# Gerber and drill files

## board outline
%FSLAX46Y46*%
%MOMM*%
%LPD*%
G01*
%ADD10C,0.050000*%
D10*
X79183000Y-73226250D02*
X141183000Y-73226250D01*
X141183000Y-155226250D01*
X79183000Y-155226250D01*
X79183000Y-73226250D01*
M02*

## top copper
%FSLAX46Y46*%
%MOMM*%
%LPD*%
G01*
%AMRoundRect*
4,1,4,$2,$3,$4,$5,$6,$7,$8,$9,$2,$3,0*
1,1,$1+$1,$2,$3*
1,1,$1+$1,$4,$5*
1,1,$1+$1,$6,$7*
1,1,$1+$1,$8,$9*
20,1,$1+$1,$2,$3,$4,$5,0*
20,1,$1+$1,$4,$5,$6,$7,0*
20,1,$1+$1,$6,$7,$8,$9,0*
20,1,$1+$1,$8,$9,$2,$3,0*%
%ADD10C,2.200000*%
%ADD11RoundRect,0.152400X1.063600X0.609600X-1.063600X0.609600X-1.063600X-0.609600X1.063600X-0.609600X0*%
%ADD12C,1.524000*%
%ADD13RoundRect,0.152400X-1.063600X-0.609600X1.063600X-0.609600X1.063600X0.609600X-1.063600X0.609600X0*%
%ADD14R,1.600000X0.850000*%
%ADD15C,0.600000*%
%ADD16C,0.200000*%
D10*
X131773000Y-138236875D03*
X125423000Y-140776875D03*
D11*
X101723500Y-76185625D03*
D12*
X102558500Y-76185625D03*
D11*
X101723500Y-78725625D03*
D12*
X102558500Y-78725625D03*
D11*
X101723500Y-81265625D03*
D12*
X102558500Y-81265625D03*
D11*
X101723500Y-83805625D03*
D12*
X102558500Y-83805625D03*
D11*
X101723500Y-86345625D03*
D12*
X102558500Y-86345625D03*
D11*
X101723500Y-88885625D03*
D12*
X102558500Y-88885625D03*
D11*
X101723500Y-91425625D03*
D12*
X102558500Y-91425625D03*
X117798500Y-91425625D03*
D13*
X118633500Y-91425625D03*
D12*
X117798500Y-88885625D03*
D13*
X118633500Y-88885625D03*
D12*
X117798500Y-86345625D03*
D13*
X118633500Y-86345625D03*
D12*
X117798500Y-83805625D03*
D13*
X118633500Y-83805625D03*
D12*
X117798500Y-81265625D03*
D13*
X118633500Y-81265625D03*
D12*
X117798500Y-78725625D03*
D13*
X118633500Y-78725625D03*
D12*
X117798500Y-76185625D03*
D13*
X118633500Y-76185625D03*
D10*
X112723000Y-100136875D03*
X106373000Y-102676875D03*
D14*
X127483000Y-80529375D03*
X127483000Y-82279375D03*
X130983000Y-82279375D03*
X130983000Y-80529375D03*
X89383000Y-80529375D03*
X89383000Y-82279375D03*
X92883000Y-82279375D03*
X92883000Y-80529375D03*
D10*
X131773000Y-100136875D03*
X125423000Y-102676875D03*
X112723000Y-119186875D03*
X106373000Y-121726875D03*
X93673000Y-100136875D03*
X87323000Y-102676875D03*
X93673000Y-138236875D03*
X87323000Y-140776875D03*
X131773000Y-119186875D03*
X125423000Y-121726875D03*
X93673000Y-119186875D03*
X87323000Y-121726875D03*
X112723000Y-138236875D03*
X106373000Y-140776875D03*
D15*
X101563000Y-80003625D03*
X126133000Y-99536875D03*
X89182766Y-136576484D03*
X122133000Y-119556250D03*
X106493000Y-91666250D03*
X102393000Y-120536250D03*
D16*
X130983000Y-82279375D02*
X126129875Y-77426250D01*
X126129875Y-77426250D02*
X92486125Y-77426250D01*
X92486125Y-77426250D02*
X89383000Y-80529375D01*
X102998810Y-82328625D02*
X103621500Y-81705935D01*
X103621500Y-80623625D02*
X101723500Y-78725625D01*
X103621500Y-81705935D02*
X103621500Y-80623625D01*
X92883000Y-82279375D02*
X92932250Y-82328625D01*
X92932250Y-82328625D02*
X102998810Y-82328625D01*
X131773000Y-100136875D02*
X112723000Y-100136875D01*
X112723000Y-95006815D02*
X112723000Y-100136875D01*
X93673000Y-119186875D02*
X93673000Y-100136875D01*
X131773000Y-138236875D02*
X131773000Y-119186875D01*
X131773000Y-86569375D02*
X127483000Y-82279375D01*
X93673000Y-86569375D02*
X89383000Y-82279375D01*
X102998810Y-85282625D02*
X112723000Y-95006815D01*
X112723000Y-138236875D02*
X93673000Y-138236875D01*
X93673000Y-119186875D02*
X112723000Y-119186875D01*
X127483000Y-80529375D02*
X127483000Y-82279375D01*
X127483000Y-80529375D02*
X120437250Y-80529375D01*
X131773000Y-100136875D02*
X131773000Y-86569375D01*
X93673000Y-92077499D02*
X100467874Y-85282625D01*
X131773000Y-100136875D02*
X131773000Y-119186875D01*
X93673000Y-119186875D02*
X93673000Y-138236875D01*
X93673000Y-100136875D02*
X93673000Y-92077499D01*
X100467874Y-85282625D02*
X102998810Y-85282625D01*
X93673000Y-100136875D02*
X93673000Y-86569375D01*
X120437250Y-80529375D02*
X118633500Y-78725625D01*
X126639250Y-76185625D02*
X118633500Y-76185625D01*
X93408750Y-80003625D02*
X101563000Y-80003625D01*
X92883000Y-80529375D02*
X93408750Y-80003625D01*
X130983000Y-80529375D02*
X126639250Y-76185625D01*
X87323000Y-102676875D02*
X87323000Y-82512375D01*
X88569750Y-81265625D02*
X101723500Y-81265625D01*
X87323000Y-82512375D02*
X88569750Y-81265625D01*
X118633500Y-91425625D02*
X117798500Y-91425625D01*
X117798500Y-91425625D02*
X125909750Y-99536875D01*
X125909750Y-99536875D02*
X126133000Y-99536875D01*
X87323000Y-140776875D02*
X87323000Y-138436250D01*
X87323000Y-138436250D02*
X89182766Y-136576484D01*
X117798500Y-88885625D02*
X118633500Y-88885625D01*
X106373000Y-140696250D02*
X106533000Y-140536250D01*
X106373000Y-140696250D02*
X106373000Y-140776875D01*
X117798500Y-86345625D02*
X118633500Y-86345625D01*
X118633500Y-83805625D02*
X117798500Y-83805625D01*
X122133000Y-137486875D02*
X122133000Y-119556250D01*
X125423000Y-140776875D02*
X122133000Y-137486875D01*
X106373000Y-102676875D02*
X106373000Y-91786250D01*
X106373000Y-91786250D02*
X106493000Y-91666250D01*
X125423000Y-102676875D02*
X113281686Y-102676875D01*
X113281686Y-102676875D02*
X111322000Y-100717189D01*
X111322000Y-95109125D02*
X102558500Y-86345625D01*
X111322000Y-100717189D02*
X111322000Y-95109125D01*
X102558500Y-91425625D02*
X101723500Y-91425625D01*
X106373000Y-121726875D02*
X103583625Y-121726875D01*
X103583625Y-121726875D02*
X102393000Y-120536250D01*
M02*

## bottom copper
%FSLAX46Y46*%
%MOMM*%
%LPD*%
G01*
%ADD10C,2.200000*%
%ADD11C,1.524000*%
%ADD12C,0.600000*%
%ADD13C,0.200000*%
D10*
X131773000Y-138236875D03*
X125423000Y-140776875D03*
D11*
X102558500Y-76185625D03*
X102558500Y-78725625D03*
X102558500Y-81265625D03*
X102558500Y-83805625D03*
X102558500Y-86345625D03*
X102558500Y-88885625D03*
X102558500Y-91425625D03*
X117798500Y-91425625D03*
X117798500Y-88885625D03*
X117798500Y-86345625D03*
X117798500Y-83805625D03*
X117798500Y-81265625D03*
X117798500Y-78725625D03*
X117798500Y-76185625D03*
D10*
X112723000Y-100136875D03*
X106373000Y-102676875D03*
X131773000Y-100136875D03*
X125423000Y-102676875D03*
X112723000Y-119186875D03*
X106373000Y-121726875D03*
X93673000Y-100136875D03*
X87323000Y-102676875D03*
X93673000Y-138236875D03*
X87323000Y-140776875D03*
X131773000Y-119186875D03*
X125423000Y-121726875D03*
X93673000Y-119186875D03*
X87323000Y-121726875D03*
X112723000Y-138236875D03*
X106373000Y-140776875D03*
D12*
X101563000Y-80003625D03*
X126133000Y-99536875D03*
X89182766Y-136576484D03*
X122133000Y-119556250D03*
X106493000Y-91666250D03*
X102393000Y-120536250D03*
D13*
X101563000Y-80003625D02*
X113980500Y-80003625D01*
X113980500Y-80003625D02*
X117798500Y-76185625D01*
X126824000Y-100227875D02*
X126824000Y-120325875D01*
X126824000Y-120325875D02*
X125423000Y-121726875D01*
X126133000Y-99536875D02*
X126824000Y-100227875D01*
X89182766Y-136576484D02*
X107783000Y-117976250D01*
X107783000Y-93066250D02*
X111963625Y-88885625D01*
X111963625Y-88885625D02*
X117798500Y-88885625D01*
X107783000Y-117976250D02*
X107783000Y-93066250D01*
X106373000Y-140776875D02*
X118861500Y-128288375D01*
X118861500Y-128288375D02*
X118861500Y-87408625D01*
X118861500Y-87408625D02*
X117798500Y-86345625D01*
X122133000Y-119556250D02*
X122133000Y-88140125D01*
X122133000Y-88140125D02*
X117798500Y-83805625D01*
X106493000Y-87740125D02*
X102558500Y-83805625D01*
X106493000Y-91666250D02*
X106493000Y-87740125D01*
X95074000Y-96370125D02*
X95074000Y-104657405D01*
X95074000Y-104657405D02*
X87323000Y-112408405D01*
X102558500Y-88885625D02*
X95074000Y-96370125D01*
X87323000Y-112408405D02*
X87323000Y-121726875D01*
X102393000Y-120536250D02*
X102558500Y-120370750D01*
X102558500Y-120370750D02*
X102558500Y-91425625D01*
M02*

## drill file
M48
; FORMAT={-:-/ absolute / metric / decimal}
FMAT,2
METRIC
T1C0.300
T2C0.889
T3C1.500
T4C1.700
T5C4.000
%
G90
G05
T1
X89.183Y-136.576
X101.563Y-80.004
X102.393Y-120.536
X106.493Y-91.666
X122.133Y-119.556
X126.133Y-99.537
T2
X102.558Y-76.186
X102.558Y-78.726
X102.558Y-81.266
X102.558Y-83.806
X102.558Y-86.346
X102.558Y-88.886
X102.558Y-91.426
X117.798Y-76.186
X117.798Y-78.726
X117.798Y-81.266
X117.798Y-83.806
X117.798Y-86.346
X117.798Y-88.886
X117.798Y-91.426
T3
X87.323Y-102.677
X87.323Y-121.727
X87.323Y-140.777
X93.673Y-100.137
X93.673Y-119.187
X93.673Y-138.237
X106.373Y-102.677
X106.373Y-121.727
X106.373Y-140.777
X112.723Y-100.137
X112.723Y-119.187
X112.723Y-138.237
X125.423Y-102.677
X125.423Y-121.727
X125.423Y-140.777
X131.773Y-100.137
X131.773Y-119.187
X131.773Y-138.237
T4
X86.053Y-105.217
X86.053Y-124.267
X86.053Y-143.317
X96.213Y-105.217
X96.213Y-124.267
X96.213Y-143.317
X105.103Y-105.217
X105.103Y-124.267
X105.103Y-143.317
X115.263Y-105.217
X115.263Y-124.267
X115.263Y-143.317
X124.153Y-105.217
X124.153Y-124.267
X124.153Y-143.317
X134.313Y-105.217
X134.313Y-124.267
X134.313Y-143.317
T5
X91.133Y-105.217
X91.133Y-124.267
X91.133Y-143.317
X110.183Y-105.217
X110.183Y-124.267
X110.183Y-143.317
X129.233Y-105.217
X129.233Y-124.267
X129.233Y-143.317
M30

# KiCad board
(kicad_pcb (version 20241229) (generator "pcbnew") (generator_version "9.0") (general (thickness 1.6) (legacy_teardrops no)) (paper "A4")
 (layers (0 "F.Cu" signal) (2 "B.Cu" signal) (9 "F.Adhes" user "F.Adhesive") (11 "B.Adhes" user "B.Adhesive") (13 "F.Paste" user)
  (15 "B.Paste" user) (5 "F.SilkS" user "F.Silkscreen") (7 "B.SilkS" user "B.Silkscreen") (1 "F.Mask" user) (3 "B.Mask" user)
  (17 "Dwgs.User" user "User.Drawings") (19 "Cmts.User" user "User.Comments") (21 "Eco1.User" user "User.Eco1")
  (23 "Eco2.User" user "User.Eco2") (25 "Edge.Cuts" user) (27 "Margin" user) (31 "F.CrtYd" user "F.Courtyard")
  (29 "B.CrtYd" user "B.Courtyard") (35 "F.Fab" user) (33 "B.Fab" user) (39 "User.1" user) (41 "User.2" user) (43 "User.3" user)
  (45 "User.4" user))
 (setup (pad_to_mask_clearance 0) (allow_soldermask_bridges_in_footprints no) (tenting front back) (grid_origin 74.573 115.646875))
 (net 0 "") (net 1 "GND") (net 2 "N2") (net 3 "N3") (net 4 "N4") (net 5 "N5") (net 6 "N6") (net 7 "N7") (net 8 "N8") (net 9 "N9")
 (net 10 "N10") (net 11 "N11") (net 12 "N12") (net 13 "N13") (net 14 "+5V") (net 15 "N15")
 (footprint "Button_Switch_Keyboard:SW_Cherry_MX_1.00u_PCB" (layer "F.Cu") (at 131.773 138.236875)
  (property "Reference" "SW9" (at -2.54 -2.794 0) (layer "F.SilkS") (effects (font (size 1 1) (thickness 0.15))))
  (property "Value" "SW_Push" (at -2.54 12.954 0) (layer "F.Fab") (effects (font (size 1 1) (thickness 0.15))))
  (pad "" np_thru_hole circle (at -7.62 5.08) (size 1.7 1.7) (drill 1.7) (layers "*.Cu" "*.Mask"))
  (pad "" np_thru_hole circle (at -2.54 5.08) (size 4 4) (drill 4) (layers "*.Cu" "*.Mask"))
  (pad "" np_thru_hole circle (at 2.54 5.08) (size 1.7 1.7) (drill 1.7) (layers "*.Cu" "*.Mask"))
  (pad "1" thru_hole circle (at 0 0) (size 2.2 2.2) (drill 1.5) (layers "*.Cu" "*.Mask") (remove_unused_layers no) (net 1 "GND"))
  (pad "2" thru_hole circle (at -6.35 2.54) (size 2.2 2.2) (drill 1.5) (layers "*.Cu" "*.Mask") (remove_unused_layers no) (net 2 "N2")))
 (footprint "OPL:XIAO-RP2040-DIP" (layer "F.Cu") (at 110.1785 83.805625)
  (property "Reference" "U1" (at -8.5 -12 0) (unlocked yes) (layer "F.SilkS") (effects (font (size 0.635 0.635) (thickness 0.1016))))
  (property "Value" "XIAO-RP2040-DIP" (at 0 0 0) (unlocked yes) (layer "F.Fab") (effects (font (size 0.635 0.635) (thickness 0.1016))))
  (pad "1" smd roundrect (at -8.455 -7.62 180) (size 2.432 1.524) (layers "F.Cu" "F.Mask") (roundrect_rratio 0.1) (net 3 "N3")
   (thermal_bridge_angle 45))
  (pad "1" thru_hole circle (at -7.62 -7.62 180) (size 1.524 1.524) (drill 0.889) (layers "*.Cu" "*.Mask") (remove_unused_layers no)
   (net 3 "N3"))
  (pad "2" smd roundrect (at -8.455 -5.08 180) (size 2.432 1.524) (layers "F.Cu" "F.Mask") (roundrect_rratio 0.1) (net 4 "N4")
   (thermal_bridge_angle 45))
  (pad "2" thru_hole circle (at -7.62 -5.08 180) (size 1.524 1.524) (drill 0.889) (layers "*.Cu" "*.Mask") (remove_unused_layers no)
   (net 4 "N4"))
  (pad "3" smd roundrect (at -8.455 -2.54 180) (size 2.432 1.524) (layers "F.Cu" "F.Mask") (roundrect_rratio 0.1) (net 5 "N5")
   (thermal_bridge_angle 45))
  (pad "3" thru_hole circle (at -7.62 -2.54 180) (size 1.524 1.524) (drill 0.889) (layers "*.Cu" "*.Mask") (remove_unused_layers no)
   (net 5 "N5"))
  (pad "4" smd roundrect (at -8.455 0 180) (size 2.432 1.524) (layers "F.Cu" "F.Mask") (roundrect_rratio 0.1) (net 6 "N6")
   (thermal_bridge_angle 45))
  (pad "4" thru_hole circle (at -7.62 0 180) (size 1.524 1.524) (drill 0.889) (layers "*.Cu" "*.Mask") (remove_unused_layers no)
   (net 6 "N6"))
  (pad "5" smd roundrect (at -8.455 2.54 180) (size 2.432 1.524) (layers "F.Cu" "F.Mask") (roundrect_rratio 0.1) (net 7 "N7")
   (thermal_bridge_angle 45))
  (pad "5" thru_hole circle (at -7.62 2.54 180) (size 1.524 1.524) (drill 0.889) (layers "*.Cu" "*.Mask") (remove_unused_layers no)
   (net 7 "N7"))
  (pad "6" smd roundrect (at -8.455 5.08 180) (size 2.432 1.524) (layers "F.Cu" "F.Mask") (roundrect_rratio 0.1) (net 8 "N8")
   (thermal_bridge_angle 45))
  (pad "6" thru_hole circle (at -7.62 5.08 180) (size 1.524 1.524) (drill 0.889) (layers "*.Cu" "*.Mask") (remove_unused_layers no)
   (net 8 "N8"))
  (pad "7" smd roundrect (at -8.455 7.62 180) (size 2.432 1.524) (layers "F.Cu" "F.Mask") (roundrect_rratio 0.1) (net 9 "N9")
   (thermal_bridge_angle 45))
  (pad "7" thru_hole circle (at -7.62 7.62 180) (size 1.524 1.524) (drill 0.889) (layers "*.Cu" "*.Mask") (remove_unused_layers no)
   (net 9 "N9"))
  (pad "8" thru_hole circle (at 7.62 7.62) (size 1.524 1.524) (drill 0.889) (layers "*.Cu" "*.Mask") (remove_unused_layers no)
   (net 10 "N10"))
  (pad "8" smd roundrect (at 8.455 7.62) (size 2.432 1.524) (layers "F.Cu" "F.Mask") (roundrect_rratio 0.1) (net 10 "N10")
   (thermal_bridge_angle 45))
  (pad "9" thru_hole circle (at 7.62 5.08) (size 1.524 1.524) (drill 0.889) (layers "*.Cu" "*.Mask") (remove_unused_layers no)
   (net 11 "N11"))
  (pad "9" smd roundrect (at 8.455 5.08) (size 2.432 1.524) (layers "F.Cu" "F.Mask") (roundrect_rratio 0.1) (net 11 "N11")
   (thermal_bridge_angle 45))
  (pad "10" thru_hole circle (at 7.62 2.54) (size 1.524 1.524) (drill 0.889) (layers "*.Cu" "*.Mask") (remove_unused_layers no)
   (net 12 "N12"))
  (pad "10" smd roundrect (at 8.455 2.54) (size 2.432 1.524) (layers "F.Cu" "F.Mask") (roundrect_rratio 0.1) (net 12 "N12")
   (thermal_bridge_angle 45))
  (pad "11" thru_hole circle (at 7.62 0) (size 1.524 1.524) (drill 0.889) (layers "*.Cu" "*.Mask") (remove_unused_layers no) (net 2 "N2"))
  (pad "11" smd roundrect (at 8.455 0) (size 2.432 1.524) (layers "F.Cu" "F.Mask") (roundrect_rratio 0.1) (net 2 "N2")
   (thermal_bridge_angle 45))
  (pad "12" thru_hole circle (at 7.62 -2.54) (size 1.524 1.524) (drill 0.889) (layers "*.Cu" "*.Mask") (remove_unused_layers no)
   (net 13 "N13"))
  (pad "12" smd roundrect (at 8.455 -2.54) (size 2.432 1.524) (layers "F.Cu" "F.Mask") (roundrect_rratio 0.1) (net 13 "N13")
   (thermal_bridge_angle 45))
  (pad "13" thru_hole circle (at 7.62 -5.08) (size 1.524 1.524) (drill 0.889) (layers "*.Cu" "*.Mask") (remove_unused_layers no)
   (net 1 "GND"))
  (pad "13" smd roundrect (at 8.455 -5.08) (size 2.432 1.524) (layers "F.Cu" "F.Mask") (roundrect_rratio 0.1) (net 1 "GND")
   (thermal_bridge_angle 45))
  (pad "14" thru_hole circle (at 7.62 -7.62) (size 1.524 1.524) (drill 0.889) (layers "*.Cu" "*.Mask") (remove_unused_layers no)
   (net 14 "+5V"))
  (pad "14" smd roundrect (at 8.455 -7.62) (size 2.432 1.524) (layers "F.Cu" "F.Mask") (roundrect_rratio 0.1) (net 14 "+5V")
   (thermal_bridge_angle 45)))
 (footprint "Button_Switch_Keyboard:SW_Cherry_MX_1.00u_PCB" (layer "F.Cu") (at 112.723 100.136875)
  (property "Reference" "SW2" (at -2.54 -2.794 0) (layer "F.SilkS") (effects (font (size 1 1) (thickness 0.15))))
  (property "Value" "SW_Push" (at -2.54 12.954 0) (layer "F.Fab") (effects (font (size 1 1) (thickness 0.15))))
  (pad "" np_thru_hole circle (at -7.62 5.08) (size 1.7 1.7) (drill 1.7) (layers "*.Cu" "*.Mask"))
  (pad "" np_thru_hole circle (at -2.54 5.08) (size 4 4) (drill 4) (layers "*.Cu" "*.Mask"))
  (pad "" np_thru_hole circle (at 2.54 5.08) (size 1.7 1.7) (drill 1.7) (layers "*.Cu" "*.Mask"))
  (pad "1" thru_hole circle (at 0 0) (size 2.2 2.2) (drill 1.5) (layers "*.Cu" "*.Mask") (remove_unused_layers no) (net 1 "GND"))
  (pad "2" thru_hole circle (at -6.35 2.54) (size 2.2 2.2) (drill 1.5) (layers "*.Cu" "*.Mask") (remove_unused_layers no) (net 6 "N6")))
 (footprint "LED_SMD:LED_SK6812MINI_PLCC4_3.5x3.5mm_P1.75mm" (layer "F.Cu") (at 129.233 81.404375)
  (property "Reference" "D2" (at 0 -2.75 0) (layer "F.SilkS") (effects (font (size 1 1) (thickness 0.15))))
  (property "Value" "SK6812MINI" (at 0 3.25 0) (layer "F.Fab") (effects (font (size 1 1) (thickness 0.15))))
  (pad "1" smd rect (at -1.75 -0.875) (size 1.6 0.85) (layers "F.Cu" "F.Mask" "F.Paste") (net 1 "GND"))
  (pad "2" smd rect (at -1.75 0.875) (size 1.6 0.85) (layers "F.Cu" "F.Mask" "F.Paste") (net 1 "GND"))
  (pad "3" smd rect (at 1.75 0.875) (size 1.6 0.85) (layers "F.Cu" "F.Mask" "F.Paste") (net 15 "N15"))
  (pad "4" smd rect (at 1.75 -0.875) (size 1.6 0.85) (layers "F.Cu" "F.Mask" "F.Paste") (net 14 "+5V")))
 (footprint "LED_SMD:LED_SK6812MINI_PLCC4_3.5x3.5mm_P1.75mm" (layer "F.Cu") (at 91.133 81.404375)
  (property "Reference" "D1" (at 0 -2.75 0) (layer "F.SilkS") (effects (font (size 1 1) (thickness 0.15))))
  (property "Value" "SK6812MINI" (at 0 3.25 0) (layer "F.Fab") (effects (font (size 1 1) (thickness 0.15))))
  (pad "1" smd rect (at -1.75 -0.875) (size 1.6 0.85) (layers "F.Cu" "F.Mask" "F.Paste") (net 15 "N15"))
  (pad "2" smd rect (at -1.75 0.875) (size 1.6 0.85) (layers "F.Cu" "F.Mask" "F.Paste") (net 1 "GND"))
  (pad "3" smd rect (at 1.75 0.875) (size 1.6 0.85) (layers "F.Cu" "F.Mask" "F.Paste") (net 4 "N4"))
  (pad "4" smd rect (at 1.75 -0.875) (size 1.6 0.85) (layers "F.Cu" "F.Mask" "F.Paste") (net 14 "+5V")))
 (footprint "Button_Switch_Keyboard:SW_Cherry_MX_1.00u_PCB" (layer "F.Cu") (at 131.773 100.136875)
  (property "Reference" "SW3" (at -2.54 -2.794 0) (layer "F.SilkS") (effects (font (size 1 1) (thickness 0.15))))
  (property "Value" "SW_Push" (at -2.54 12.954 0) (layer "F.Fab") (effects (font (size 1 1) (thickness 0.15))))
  (pad "" np_thru_hole circle (at -7.62 5.08) (size 1.7 1.7) (drill 1.7) (layers "*.Cu" "*.Mask"))
  (pad "" np_thru_hole circle (at -2.54 5.08) (size 4 4) (drill 4) (layers "*.Cu" "*.Mask"))
  (pad "" np_thru_hole circle (at 2.54 5.08) (size 1.7 1.7) (drill 1.7) (layers "*.Cu" "*.Mask"))
  (pad "1" thru_hole circle (at 0 0) (size 2.2 2.2) (drill 1.5) (layers "*.Cu" "*.Mask") (remove_unused_layers no) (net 1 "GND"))
  (pad "2" thru_hole circle (at -6.35 2.54) (size 2.2 2.2) (drill 1.5) (layers "*.Cu" "*.Mask") (remove_unused_layers no) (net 7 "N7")))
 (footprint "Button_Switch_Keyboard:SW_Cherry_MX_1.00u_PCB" (layer "F.Cu") (at 112.723 119.186875)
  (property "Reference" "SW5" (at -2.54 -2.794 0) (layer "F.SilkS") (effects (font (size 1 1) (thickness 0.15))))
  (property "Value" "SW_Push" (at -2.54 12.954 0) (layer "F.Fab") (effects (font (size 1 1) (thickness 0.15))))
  (pad "" np_thru_hole circle (at -7.62 5.08) (size 1.7 1.7) (drill 1.7) (layers "*.Cu" "*.Mask"))
  (pad "" np_thru_hole circle (at -2.54 5.08) (size 4 4) (drill 4) (layers "*.Cu" "*.Mask"))
  (pad "" np_thru_hole circle (at 2.54 5.08) (size 1.7 1.7) (drill 1.7) (layers "*.Cu" "*.Mask"))
  (pad "1" thru_hole circle (at 0 0) (size 2.2 2.2) (drill 1.5) (layers "*.Cu" "*.Mask") (remove_unused_layers no) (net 1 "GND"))
  (pad "2" thru_hole circle (at -6.35 2.54) (size 2.2 2.2) (drill 1.5) (layers "*.Cu" "*.Mask") (remove_unused_layers no) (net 9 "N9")))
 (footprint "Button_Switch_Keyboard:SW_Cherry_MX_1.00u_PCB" (layer "F.Cu") (at 93.673 100.136875)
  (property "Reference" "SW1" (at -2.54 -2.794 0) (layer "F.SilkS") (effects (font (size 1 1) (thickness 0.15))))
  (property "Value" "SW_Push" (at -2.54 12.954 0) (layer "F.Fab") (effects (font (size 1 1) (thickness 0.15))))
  (pad "" np_thru_hole circle (at -7.62 5.08) (size 1.7 1.7) (drill 1.7) (layers "*.Cu" "*.Mask"))
  (pad "" np_thru_hole circle (at -2.54 5.08) (size 4 4) (drill 4) (layers "*.Cu" "*.Mask"))
  (pad "" np_thru_hole circle (at 2.54 5.08) (size 1.7 1.7) (drill 1.7) (layers "*.Cu" "*.Mask"))
  (pad "1" thru_hole circle (at 0 0) (size 2.2 2.2) (drill 1.5) (layers "*.Cu" "*.Mask") (remove_unused_layers no) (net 1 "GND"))
  (pad "2" thru_hole circle (at -6.35 2.54) (size 2.2 2.2) (drill 1.5) (layers "*.Cu" "*.Mask") (remove_unused_layers no) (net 5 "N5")))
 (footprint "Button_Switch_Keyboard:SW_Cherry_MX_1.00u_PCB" (layer "F.Cu") (at 93.673 138.236875)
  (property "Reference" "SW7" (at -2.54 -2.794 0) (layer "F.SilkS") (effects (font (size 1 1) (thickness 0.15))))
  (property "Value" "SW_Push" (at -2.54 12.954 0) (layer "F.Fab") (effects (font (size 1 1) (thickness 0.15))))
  (pad "" np_thru_hole circle (at -7.62 5.08) (size 1.7 1.7) (drill 1.7) (layers "*.Cu" "*.Mask"))
  (pad "" np_thru_hole circle (at -2.54 5.08) (size 4 4) (drill 4) (layers "*.Cu" "*.Mask"))
  (pad "" np_thru_hole circle (at 2.54 5.08) (size 1.7 1.7) (drill 1.7) (layers "*.Cu" "*.Mask"))
  (pad "1" thru_hole circle (at 0 0) (size 2.2 2.2) (drill 1.5) (layers "*.Cu" "*.Mask") (remove_unused_layers no) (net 1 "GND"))
  (pad "2" thru_hole circle (at -6.35 2.54) (size 2.2 2.2) (drill 1.5) (layers "*.Cu" "*.Mask") (remove_unused_layers no) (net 11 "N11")))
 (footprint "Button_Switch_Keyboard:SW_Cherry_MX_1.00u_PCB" (layer "F.Cu") (at 131.773 119.186875)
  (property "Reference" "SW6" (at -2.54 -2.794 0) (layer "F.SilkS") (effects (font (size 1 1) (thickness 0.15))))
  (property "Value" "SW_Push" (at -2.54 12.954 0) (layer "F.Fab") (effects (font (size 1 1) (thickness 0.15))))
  (pad "" np_thru_hole circle (at -7.62 5.08) (size 1.7 1.7) (drill 1.7) (layers "*.Cu" "*.Mask"))
  (pad "" np_thru_hole circle (at -2.54 5.08) (size 4 4) (drill 4) (layers "*.Cu" "*.Mask"))
  (pad "" np_thru_hole circle (at 2.54 5.08) (size 1.7 1.7) (drill 1.7) (layers "*.Cu" "*.Mask"))
  (pad "1" thru_hole circle (at 0 0) (size 2.2 2.2) (drill 1.5) (layers "*.Cu" "*.Mask") (remove_unused_layers no) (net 1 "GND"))
  (pad "2" thru_hole circle (at -6.35 2.54) (size 2.2 2.2) (drill 1.5) (layers "*.Cu" "*.Mask") (remove_unused_layers no) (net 10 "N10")))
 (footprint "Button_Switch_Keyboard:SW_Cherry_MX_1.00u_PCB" (layer "F.Cu") (at 93.673 119.186875)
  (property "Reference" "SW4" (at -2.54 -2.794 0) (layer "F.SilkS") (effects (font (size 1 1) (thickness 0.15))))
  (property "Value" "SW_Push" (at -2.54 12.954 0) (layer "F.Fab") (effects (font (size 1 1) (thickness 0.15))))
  (pad "" np_thru_hole circle (at -7.62 5.08) (size 1.7 1.7) (drill 1.7) (layers "*.Cu" "*.Mask"))
  (pad "" np_thru_hole circle (at -2.54 5.08) (size 4 4) (drill 4) (layers "*.Cu" "*.Mask"))
  (pad "" np_thru_hole circle (at 2.54 5.08) (size 1.7 1.7) (drill 1.7) (layers "*.Cu" "*.Mask"))
  (pad "1" thru_hole circle (at 0 0) (size 2.2 2.2) (drill 1.5) (layers "*.Cu" "*.Mask") (remove_unused_layers no) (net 1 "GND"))
  (pad "2" thru_hole circle (at -6.35 2.54) (size 2.2 2.2) (drill 1.5) (layers "*.Cu" "*.Mask") (remove_unused_layers no) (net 8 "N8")))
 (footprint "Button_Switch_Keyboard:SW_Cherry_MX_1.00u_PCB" (layer "F.Cu") (at 112.723 138.236875)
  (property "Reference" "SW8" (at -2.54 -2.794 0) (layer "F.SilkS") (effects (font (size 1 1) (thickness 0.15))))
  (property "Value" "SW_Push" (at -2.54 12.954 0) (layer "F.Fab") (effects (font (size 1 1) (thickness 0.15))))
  (pad "" np_thru_hole circle (at -7.62 5.08) (size 1.7 1.7) (drill 1.7) (layers "*.Cu" "*.Mask"))
  (pad "" np_thru_hole circle (at -2.54 5.08) (size 4 4) (drill 4) (layers "*.Cu" "*.Mask"))
  (pad "" np_thru_hole circle (at 2.54 5.08) (size 1.7 1.7) (drill 1.7) (layers "*.Cu" "*.Mask"))
  (pad "1" thru_hole circle (at 0 0) (size 2.2 2.2) (drill 1.5) (layers "*.Cu" "*.Mask") (remove_unused_layers no) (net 1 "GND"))
  (pad "2" thru_hole circle (at -6.35 2.54) (size 2.2 2.2) (drill 1.5) (layers "*.Cu" "*.Mask") (remove_unused_layers no) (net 12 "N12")))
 (gr_rect (start 79.183 73.22625) (end 141.183 155.22625) (stroke (width 0.05) (type solid)) (fill no) (layer "Edge.Cuts"))
 (segment (start 130.983 82.279375) (end 126.129875 77.42625) (width 0.2) (layer "F.Cu") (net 15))
 (segment (start 126.129875 77.42625) (end 92.486125 77.42625) (width 0.2) (layer "F.Cu") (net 15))
 (segment (start 92.486125 77.42625) (end 89.383 80.529375) (width 0.2) (layer "F.Cu") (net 15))
 (segment (start 102.99881 82.328625) (end 103.6215 81.705935) (width 0.2) (layer "F.Cu") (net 4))
 (segment (start 103.6215 80.623625) (end 101.7235 78.725625) (width 0.2) (layer "F.Cu") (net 4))
 (segment (start 103.6215 81.705935) (end 103.6215 80.623625) (width 0.2) (layer "F.Cu") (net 4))
 (segment (start 92.883 82.279375) (end 92.93225 82.328625) (width 0.2) (layer "F.Cu") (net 4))
 (segment (start 92.93225 82.328625) (end 102.99881 82.328625) (width 0.2) (layer "F.Cu") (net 4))
 (segment (start 131.773 100.136875) (end 112.723 100.136875) (width 0.2) (layer "F.Cu") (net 1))
 (segment (start 112.723 95.006815) (end 112.723 100.136875) (width 0.2) (layer "F.Cu") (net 1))
 (segment (start 93.673 119.186875) (end 93.673 100.136875) (width 0.2) (layer "F.Cu") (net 1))
 (segment (start 131.773 138.236875) (end 131.773 119.186875) (width 0.2) (layer "F.Cu") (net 1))
 (segment (start 131.773 86.569375) (end 127.483 82.279375) (width 0.2) (layer "F.Cu") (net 1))
 (segment (start 93.673 86.569375) (end 89.383 82.279375) (width 0.2) (layer "F.Cu") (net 1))
 (segment (start 102.99881 85.282625) (end 112.723 95.006815) (width 0.2) (layer "F.Cu") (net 1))
 (segment (start 112.723 138.236875) (end 93.673 138.236875) (width 0.2) (layer "F.Cu") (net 1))
 (segment (start 93.673 119.186875) (end 112.723 119.186875) (width 0.2) (layer "F.Cu") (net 1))
 (segment (start 127.483 80.529375) (end 127.483 82.279375) (width 0.2) (layer "F.Cu") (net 1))
 (segment (start 127.483 80.529375) (end 120.43725 80.529375) (width 0.2) (layer "F.Cu") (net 1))
 (segment (start 131.773 100.136875) (end 131.773 86.569375) (width 0.2) (layer "F.Cu") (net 1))
 (segment (start 93.673 92.077499) (end 100.467874 85.282625) (width 0.2) (layer "F.Cu") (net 1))
 (segment (start 131.773 100.136875) (end 131.773 119.186875) (width 0.2) (layer "F.Cu") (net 1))
 (segment (start 93.673 119.186875) (end 93.673 138.236875) (width 0.2) (layer "F.Cu") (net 1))
 (segment (start 93.673 100.136875) (end 93.673 92.077499) (width 0.2) (layer "F.Cu") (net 1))
 (segment (start 100.467874 85.282625) (end 102.99881 85.282625) (width 0.2) (layer "F.Cu") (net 1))
 (segment (start 93.673 100.136875) (end 93.673 86.569375) (width 0.2) (layer "F.Cu") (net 1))
 (segment (start 120.43725 80.529375) (end 118.6335 78.725625) (width 0.2) (layer "F.Cu") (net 1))
 (segment (start 126.63925 76.185625) (end 118.6335 76.185625) (width 0.2) (layer "F.Cu") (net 14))
 (segment (start 93.40875 80.003625) (end 101.563 80.003625) (width 0.2) (layer "F.Cu") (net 14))
 (segment (start 92.883 80.529375) (end 93.40875 80.003625) (width 0.2) (layer "F.Cu") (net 14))
 (segment (start 130.983 80.529375) (end 126.63925 76.185625) (width 0.2) (layer "F.Cu") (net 14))
 (via (at 101.563 80.003625) (size 0.6) (drill 0.3) (layers "F.Cu" "B.Cu") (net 14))
 (segment (start 101.563 80.003625) (end 113.9805 80.003625) (width 0.2) (layer "B.Cu") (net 14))
 (segment (start 113.9805 80.003625) (end 117.7985 76.185625) (width 0.2) (layer "B.Cu") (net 14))
 (segment (start 87.323 102.676875) (end 87.323 82.512375) (width 0.2) (layer "F.Cu") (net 5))
 (segment (start 88.56975 81.265625) (end 101.7235 81.265625) (width 0.2) (layer "F.Cu") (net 5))
 (segment (start 87.323 82.512375) (end 88.56975 81.265625) (width 0.2) (layer "F.Cu") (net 5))
 (segment (start 118.6335 91.425625) (end 117.7985 91.425625) (width 0.2) (layer "F.Cu") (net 10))
 (segment (start 117.7985 91.425625) (end 125.90975 99.536875) (width 0.2) (layer "F.Cu") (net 10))
 (segment (start 125.90975 99.536875) (end 126.133 99.536875) (width 0.2) (layer "F.Cu") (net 10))
 (via (at 126.133 99.536875) (size 0.6) (drill 0.3) (layers "F.Cu" "B.Cu") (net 10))
 (segment (start 126.824 100.227875) (end 126.824 120.325875) (width 0.2) (layer "B.Cu") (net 10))
 (segment (start 126.824 120.325875) (end 125.423 121.726875) (width 0.2) (layer "B.Cu") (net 10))
 (segment (start 126.133 99.536875) (end 126.824 100.227875) (width 0.2) (layer "B.Cu") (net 10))
 (segment (start 87.323 140.776875) (end 87.323 138.43625) (width 0.2) (layer "F.Cu") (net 11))
 (segment (start 87.323 138.43625) (end 89.182766 136.576484) (width 0.2) (layer "F.Cu") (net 11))
 (segment (start 117.7985 88.885625) (end 118.6335 88.885625) (width 0.2) (layer "F.Cu") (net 11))
 (via (at 89.182766 136.576484) (size 0.6) (drill 0.3) (layers "F.Cu" "B.Cu") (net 11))
 (segment (start 89.182766 136.576484) (end 107.783 117.97625) (width 0.2) (layer "B.Cu") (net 11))
 (segment (start 107.783 93.06625) (end 111.963625 88.885625) (width 0.2) (layer "B.Cu") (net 11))
 (segment (start 111.963625 88.885625) (end 117.7985 88.885625) (width 0.2) (layer "B.Cu") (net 11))
 (segment (start 107.783 117.97625) (end 107.783 93.06625) (width 0.2) (layer "B.Cu") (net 11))
 (segment (start 106.373 140.69625) (end 106.533 140.53625) (width 0.2) (layer "F.Cu") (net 12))
 (segment (start 106.373 140.69625) (end 106.373 140.776875) (width 0.2) (layer "F.Cu") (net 12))
 (segment (start 117.7985 86.345625) (end 118.6335 86.345625) (width 0.2) (layer "F.Cu") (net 12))
 (segment (start 106.373 140.776875) (end 118.8615 128.288375) (width 0.2) (layer "B.Cu") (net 12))
 (segment (start 118.8615 128.288375) (end 118.8615 87.408625) (width 0.2) (layer "B.Cu") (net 12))
 (segment (start 118.8615 87.408625) (end 117.7985 86.345625) (width 0.2) (layer "B.Cu") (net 12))
 (segment (start 118.6335 83.805625) (end 117.7985 83.805625) (width 0.2) (layer "F.Cu") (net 2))
 (segment (start 122.133 137.486875) (end 122.133 119.55625) (width 0.2) (layer "F.Cu") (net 2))
 (segment (start 125.423 140.776875) (end 122.133 137.486875) (width 0.2) (layer "F.Cu") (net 2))
 (via (at 122.133 119.55625) (size 0.6) (drill 0.3) (layers "F.Cu" "B.Cu") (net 2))
 (segment (start 122.133 119.55625) (end 122.133 88.140125) (width 0.2) (layer "B.Cu") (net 2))
 (segment (start 122.133 88.140125) (end 117.7985 83.805625) (width 0.2) (layer "B.Cu") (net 2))
 (segment (start 106.373 102.676875) (end 106.373 91.78625) (width 0.2) (layer "F.Cu") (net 6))
 (segment (start 106.373 91.78625) (end 106.493 91.66625) (width 0.2) (layer "F.Cu") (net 6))
 (via (at 106.493 91.66625) (size 0.6) (drill 0.3) (layers "F.Cu" "B.Cu") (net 6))
 (segment (start 106.493 87.740125) (end 102.5585 83.805625) (width 0.2) (layer "B.Cu") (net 6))
 (segment (start 106.493 91.66625) (end 106.493 87.740125) (width 0.2) (layer "B.Cu") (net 6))
 (segment (start 125.423 102.676875) (end 113.281686 102.676875) (width 0.2) (layer "F.Cu") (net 7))
 (segment (start 113.281686 102.676875) (end 111.322 100.717189) (width 0.2) (layer "F.Cu") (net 7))
 (segment (start 111.322 95.109125) (end 102.5585 86.345625) (width 0.2) (layer "F.Cu") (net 7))
 (segment (start 111.322 100.717189) (end 111.322 95.109125) (width 0.2) (layer "F.Cu") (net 7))
 (segment (start 95.074 96.370125) (end 95.074 104.657405) (width 0.2) (layer "B.Cu") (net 8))
 (segment (start 95.074 104.657405) (end 87.323 112.408405) (width 0.2) (layer "B.Cu") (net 8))
 (segment (start 102.5585 88.885625) (end 95.074 96.370125) (width 0.2) (layer "B.Cu") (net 8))
 (segment (start 87.323 112.408405) (end 87.323 121.726875) (width 0.2) (layer "B.Cu") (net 8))
 (segment (start 102.5585 91.425625) (end 101.7235 91.425625) (width 0.2) (layer "F.Cu") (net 9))
 (segment (start 106.373 121.726875) (end 103.583625 121.726875) (width 0.2) (layer "F.Cu") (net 9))
 (segment (start 103.583625 121.726875) (end 102.393 120.53625) (width 0.2) (layer "F.Cu") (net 9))
 (via (at 102.393 120.53625) (size 0.6) (drill 0.3) (layers "F.Cu" "B.Cu") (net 9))
 (segment (start 102.393 120.53625) (end 102.5585 120.37075) (width 0.2) (layer "B.Cu") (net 9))
 (segment (start 102.5585 120.37075) (end 102.5585 91.425625) (width 0.2) (layer "B.Cu") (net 9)))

